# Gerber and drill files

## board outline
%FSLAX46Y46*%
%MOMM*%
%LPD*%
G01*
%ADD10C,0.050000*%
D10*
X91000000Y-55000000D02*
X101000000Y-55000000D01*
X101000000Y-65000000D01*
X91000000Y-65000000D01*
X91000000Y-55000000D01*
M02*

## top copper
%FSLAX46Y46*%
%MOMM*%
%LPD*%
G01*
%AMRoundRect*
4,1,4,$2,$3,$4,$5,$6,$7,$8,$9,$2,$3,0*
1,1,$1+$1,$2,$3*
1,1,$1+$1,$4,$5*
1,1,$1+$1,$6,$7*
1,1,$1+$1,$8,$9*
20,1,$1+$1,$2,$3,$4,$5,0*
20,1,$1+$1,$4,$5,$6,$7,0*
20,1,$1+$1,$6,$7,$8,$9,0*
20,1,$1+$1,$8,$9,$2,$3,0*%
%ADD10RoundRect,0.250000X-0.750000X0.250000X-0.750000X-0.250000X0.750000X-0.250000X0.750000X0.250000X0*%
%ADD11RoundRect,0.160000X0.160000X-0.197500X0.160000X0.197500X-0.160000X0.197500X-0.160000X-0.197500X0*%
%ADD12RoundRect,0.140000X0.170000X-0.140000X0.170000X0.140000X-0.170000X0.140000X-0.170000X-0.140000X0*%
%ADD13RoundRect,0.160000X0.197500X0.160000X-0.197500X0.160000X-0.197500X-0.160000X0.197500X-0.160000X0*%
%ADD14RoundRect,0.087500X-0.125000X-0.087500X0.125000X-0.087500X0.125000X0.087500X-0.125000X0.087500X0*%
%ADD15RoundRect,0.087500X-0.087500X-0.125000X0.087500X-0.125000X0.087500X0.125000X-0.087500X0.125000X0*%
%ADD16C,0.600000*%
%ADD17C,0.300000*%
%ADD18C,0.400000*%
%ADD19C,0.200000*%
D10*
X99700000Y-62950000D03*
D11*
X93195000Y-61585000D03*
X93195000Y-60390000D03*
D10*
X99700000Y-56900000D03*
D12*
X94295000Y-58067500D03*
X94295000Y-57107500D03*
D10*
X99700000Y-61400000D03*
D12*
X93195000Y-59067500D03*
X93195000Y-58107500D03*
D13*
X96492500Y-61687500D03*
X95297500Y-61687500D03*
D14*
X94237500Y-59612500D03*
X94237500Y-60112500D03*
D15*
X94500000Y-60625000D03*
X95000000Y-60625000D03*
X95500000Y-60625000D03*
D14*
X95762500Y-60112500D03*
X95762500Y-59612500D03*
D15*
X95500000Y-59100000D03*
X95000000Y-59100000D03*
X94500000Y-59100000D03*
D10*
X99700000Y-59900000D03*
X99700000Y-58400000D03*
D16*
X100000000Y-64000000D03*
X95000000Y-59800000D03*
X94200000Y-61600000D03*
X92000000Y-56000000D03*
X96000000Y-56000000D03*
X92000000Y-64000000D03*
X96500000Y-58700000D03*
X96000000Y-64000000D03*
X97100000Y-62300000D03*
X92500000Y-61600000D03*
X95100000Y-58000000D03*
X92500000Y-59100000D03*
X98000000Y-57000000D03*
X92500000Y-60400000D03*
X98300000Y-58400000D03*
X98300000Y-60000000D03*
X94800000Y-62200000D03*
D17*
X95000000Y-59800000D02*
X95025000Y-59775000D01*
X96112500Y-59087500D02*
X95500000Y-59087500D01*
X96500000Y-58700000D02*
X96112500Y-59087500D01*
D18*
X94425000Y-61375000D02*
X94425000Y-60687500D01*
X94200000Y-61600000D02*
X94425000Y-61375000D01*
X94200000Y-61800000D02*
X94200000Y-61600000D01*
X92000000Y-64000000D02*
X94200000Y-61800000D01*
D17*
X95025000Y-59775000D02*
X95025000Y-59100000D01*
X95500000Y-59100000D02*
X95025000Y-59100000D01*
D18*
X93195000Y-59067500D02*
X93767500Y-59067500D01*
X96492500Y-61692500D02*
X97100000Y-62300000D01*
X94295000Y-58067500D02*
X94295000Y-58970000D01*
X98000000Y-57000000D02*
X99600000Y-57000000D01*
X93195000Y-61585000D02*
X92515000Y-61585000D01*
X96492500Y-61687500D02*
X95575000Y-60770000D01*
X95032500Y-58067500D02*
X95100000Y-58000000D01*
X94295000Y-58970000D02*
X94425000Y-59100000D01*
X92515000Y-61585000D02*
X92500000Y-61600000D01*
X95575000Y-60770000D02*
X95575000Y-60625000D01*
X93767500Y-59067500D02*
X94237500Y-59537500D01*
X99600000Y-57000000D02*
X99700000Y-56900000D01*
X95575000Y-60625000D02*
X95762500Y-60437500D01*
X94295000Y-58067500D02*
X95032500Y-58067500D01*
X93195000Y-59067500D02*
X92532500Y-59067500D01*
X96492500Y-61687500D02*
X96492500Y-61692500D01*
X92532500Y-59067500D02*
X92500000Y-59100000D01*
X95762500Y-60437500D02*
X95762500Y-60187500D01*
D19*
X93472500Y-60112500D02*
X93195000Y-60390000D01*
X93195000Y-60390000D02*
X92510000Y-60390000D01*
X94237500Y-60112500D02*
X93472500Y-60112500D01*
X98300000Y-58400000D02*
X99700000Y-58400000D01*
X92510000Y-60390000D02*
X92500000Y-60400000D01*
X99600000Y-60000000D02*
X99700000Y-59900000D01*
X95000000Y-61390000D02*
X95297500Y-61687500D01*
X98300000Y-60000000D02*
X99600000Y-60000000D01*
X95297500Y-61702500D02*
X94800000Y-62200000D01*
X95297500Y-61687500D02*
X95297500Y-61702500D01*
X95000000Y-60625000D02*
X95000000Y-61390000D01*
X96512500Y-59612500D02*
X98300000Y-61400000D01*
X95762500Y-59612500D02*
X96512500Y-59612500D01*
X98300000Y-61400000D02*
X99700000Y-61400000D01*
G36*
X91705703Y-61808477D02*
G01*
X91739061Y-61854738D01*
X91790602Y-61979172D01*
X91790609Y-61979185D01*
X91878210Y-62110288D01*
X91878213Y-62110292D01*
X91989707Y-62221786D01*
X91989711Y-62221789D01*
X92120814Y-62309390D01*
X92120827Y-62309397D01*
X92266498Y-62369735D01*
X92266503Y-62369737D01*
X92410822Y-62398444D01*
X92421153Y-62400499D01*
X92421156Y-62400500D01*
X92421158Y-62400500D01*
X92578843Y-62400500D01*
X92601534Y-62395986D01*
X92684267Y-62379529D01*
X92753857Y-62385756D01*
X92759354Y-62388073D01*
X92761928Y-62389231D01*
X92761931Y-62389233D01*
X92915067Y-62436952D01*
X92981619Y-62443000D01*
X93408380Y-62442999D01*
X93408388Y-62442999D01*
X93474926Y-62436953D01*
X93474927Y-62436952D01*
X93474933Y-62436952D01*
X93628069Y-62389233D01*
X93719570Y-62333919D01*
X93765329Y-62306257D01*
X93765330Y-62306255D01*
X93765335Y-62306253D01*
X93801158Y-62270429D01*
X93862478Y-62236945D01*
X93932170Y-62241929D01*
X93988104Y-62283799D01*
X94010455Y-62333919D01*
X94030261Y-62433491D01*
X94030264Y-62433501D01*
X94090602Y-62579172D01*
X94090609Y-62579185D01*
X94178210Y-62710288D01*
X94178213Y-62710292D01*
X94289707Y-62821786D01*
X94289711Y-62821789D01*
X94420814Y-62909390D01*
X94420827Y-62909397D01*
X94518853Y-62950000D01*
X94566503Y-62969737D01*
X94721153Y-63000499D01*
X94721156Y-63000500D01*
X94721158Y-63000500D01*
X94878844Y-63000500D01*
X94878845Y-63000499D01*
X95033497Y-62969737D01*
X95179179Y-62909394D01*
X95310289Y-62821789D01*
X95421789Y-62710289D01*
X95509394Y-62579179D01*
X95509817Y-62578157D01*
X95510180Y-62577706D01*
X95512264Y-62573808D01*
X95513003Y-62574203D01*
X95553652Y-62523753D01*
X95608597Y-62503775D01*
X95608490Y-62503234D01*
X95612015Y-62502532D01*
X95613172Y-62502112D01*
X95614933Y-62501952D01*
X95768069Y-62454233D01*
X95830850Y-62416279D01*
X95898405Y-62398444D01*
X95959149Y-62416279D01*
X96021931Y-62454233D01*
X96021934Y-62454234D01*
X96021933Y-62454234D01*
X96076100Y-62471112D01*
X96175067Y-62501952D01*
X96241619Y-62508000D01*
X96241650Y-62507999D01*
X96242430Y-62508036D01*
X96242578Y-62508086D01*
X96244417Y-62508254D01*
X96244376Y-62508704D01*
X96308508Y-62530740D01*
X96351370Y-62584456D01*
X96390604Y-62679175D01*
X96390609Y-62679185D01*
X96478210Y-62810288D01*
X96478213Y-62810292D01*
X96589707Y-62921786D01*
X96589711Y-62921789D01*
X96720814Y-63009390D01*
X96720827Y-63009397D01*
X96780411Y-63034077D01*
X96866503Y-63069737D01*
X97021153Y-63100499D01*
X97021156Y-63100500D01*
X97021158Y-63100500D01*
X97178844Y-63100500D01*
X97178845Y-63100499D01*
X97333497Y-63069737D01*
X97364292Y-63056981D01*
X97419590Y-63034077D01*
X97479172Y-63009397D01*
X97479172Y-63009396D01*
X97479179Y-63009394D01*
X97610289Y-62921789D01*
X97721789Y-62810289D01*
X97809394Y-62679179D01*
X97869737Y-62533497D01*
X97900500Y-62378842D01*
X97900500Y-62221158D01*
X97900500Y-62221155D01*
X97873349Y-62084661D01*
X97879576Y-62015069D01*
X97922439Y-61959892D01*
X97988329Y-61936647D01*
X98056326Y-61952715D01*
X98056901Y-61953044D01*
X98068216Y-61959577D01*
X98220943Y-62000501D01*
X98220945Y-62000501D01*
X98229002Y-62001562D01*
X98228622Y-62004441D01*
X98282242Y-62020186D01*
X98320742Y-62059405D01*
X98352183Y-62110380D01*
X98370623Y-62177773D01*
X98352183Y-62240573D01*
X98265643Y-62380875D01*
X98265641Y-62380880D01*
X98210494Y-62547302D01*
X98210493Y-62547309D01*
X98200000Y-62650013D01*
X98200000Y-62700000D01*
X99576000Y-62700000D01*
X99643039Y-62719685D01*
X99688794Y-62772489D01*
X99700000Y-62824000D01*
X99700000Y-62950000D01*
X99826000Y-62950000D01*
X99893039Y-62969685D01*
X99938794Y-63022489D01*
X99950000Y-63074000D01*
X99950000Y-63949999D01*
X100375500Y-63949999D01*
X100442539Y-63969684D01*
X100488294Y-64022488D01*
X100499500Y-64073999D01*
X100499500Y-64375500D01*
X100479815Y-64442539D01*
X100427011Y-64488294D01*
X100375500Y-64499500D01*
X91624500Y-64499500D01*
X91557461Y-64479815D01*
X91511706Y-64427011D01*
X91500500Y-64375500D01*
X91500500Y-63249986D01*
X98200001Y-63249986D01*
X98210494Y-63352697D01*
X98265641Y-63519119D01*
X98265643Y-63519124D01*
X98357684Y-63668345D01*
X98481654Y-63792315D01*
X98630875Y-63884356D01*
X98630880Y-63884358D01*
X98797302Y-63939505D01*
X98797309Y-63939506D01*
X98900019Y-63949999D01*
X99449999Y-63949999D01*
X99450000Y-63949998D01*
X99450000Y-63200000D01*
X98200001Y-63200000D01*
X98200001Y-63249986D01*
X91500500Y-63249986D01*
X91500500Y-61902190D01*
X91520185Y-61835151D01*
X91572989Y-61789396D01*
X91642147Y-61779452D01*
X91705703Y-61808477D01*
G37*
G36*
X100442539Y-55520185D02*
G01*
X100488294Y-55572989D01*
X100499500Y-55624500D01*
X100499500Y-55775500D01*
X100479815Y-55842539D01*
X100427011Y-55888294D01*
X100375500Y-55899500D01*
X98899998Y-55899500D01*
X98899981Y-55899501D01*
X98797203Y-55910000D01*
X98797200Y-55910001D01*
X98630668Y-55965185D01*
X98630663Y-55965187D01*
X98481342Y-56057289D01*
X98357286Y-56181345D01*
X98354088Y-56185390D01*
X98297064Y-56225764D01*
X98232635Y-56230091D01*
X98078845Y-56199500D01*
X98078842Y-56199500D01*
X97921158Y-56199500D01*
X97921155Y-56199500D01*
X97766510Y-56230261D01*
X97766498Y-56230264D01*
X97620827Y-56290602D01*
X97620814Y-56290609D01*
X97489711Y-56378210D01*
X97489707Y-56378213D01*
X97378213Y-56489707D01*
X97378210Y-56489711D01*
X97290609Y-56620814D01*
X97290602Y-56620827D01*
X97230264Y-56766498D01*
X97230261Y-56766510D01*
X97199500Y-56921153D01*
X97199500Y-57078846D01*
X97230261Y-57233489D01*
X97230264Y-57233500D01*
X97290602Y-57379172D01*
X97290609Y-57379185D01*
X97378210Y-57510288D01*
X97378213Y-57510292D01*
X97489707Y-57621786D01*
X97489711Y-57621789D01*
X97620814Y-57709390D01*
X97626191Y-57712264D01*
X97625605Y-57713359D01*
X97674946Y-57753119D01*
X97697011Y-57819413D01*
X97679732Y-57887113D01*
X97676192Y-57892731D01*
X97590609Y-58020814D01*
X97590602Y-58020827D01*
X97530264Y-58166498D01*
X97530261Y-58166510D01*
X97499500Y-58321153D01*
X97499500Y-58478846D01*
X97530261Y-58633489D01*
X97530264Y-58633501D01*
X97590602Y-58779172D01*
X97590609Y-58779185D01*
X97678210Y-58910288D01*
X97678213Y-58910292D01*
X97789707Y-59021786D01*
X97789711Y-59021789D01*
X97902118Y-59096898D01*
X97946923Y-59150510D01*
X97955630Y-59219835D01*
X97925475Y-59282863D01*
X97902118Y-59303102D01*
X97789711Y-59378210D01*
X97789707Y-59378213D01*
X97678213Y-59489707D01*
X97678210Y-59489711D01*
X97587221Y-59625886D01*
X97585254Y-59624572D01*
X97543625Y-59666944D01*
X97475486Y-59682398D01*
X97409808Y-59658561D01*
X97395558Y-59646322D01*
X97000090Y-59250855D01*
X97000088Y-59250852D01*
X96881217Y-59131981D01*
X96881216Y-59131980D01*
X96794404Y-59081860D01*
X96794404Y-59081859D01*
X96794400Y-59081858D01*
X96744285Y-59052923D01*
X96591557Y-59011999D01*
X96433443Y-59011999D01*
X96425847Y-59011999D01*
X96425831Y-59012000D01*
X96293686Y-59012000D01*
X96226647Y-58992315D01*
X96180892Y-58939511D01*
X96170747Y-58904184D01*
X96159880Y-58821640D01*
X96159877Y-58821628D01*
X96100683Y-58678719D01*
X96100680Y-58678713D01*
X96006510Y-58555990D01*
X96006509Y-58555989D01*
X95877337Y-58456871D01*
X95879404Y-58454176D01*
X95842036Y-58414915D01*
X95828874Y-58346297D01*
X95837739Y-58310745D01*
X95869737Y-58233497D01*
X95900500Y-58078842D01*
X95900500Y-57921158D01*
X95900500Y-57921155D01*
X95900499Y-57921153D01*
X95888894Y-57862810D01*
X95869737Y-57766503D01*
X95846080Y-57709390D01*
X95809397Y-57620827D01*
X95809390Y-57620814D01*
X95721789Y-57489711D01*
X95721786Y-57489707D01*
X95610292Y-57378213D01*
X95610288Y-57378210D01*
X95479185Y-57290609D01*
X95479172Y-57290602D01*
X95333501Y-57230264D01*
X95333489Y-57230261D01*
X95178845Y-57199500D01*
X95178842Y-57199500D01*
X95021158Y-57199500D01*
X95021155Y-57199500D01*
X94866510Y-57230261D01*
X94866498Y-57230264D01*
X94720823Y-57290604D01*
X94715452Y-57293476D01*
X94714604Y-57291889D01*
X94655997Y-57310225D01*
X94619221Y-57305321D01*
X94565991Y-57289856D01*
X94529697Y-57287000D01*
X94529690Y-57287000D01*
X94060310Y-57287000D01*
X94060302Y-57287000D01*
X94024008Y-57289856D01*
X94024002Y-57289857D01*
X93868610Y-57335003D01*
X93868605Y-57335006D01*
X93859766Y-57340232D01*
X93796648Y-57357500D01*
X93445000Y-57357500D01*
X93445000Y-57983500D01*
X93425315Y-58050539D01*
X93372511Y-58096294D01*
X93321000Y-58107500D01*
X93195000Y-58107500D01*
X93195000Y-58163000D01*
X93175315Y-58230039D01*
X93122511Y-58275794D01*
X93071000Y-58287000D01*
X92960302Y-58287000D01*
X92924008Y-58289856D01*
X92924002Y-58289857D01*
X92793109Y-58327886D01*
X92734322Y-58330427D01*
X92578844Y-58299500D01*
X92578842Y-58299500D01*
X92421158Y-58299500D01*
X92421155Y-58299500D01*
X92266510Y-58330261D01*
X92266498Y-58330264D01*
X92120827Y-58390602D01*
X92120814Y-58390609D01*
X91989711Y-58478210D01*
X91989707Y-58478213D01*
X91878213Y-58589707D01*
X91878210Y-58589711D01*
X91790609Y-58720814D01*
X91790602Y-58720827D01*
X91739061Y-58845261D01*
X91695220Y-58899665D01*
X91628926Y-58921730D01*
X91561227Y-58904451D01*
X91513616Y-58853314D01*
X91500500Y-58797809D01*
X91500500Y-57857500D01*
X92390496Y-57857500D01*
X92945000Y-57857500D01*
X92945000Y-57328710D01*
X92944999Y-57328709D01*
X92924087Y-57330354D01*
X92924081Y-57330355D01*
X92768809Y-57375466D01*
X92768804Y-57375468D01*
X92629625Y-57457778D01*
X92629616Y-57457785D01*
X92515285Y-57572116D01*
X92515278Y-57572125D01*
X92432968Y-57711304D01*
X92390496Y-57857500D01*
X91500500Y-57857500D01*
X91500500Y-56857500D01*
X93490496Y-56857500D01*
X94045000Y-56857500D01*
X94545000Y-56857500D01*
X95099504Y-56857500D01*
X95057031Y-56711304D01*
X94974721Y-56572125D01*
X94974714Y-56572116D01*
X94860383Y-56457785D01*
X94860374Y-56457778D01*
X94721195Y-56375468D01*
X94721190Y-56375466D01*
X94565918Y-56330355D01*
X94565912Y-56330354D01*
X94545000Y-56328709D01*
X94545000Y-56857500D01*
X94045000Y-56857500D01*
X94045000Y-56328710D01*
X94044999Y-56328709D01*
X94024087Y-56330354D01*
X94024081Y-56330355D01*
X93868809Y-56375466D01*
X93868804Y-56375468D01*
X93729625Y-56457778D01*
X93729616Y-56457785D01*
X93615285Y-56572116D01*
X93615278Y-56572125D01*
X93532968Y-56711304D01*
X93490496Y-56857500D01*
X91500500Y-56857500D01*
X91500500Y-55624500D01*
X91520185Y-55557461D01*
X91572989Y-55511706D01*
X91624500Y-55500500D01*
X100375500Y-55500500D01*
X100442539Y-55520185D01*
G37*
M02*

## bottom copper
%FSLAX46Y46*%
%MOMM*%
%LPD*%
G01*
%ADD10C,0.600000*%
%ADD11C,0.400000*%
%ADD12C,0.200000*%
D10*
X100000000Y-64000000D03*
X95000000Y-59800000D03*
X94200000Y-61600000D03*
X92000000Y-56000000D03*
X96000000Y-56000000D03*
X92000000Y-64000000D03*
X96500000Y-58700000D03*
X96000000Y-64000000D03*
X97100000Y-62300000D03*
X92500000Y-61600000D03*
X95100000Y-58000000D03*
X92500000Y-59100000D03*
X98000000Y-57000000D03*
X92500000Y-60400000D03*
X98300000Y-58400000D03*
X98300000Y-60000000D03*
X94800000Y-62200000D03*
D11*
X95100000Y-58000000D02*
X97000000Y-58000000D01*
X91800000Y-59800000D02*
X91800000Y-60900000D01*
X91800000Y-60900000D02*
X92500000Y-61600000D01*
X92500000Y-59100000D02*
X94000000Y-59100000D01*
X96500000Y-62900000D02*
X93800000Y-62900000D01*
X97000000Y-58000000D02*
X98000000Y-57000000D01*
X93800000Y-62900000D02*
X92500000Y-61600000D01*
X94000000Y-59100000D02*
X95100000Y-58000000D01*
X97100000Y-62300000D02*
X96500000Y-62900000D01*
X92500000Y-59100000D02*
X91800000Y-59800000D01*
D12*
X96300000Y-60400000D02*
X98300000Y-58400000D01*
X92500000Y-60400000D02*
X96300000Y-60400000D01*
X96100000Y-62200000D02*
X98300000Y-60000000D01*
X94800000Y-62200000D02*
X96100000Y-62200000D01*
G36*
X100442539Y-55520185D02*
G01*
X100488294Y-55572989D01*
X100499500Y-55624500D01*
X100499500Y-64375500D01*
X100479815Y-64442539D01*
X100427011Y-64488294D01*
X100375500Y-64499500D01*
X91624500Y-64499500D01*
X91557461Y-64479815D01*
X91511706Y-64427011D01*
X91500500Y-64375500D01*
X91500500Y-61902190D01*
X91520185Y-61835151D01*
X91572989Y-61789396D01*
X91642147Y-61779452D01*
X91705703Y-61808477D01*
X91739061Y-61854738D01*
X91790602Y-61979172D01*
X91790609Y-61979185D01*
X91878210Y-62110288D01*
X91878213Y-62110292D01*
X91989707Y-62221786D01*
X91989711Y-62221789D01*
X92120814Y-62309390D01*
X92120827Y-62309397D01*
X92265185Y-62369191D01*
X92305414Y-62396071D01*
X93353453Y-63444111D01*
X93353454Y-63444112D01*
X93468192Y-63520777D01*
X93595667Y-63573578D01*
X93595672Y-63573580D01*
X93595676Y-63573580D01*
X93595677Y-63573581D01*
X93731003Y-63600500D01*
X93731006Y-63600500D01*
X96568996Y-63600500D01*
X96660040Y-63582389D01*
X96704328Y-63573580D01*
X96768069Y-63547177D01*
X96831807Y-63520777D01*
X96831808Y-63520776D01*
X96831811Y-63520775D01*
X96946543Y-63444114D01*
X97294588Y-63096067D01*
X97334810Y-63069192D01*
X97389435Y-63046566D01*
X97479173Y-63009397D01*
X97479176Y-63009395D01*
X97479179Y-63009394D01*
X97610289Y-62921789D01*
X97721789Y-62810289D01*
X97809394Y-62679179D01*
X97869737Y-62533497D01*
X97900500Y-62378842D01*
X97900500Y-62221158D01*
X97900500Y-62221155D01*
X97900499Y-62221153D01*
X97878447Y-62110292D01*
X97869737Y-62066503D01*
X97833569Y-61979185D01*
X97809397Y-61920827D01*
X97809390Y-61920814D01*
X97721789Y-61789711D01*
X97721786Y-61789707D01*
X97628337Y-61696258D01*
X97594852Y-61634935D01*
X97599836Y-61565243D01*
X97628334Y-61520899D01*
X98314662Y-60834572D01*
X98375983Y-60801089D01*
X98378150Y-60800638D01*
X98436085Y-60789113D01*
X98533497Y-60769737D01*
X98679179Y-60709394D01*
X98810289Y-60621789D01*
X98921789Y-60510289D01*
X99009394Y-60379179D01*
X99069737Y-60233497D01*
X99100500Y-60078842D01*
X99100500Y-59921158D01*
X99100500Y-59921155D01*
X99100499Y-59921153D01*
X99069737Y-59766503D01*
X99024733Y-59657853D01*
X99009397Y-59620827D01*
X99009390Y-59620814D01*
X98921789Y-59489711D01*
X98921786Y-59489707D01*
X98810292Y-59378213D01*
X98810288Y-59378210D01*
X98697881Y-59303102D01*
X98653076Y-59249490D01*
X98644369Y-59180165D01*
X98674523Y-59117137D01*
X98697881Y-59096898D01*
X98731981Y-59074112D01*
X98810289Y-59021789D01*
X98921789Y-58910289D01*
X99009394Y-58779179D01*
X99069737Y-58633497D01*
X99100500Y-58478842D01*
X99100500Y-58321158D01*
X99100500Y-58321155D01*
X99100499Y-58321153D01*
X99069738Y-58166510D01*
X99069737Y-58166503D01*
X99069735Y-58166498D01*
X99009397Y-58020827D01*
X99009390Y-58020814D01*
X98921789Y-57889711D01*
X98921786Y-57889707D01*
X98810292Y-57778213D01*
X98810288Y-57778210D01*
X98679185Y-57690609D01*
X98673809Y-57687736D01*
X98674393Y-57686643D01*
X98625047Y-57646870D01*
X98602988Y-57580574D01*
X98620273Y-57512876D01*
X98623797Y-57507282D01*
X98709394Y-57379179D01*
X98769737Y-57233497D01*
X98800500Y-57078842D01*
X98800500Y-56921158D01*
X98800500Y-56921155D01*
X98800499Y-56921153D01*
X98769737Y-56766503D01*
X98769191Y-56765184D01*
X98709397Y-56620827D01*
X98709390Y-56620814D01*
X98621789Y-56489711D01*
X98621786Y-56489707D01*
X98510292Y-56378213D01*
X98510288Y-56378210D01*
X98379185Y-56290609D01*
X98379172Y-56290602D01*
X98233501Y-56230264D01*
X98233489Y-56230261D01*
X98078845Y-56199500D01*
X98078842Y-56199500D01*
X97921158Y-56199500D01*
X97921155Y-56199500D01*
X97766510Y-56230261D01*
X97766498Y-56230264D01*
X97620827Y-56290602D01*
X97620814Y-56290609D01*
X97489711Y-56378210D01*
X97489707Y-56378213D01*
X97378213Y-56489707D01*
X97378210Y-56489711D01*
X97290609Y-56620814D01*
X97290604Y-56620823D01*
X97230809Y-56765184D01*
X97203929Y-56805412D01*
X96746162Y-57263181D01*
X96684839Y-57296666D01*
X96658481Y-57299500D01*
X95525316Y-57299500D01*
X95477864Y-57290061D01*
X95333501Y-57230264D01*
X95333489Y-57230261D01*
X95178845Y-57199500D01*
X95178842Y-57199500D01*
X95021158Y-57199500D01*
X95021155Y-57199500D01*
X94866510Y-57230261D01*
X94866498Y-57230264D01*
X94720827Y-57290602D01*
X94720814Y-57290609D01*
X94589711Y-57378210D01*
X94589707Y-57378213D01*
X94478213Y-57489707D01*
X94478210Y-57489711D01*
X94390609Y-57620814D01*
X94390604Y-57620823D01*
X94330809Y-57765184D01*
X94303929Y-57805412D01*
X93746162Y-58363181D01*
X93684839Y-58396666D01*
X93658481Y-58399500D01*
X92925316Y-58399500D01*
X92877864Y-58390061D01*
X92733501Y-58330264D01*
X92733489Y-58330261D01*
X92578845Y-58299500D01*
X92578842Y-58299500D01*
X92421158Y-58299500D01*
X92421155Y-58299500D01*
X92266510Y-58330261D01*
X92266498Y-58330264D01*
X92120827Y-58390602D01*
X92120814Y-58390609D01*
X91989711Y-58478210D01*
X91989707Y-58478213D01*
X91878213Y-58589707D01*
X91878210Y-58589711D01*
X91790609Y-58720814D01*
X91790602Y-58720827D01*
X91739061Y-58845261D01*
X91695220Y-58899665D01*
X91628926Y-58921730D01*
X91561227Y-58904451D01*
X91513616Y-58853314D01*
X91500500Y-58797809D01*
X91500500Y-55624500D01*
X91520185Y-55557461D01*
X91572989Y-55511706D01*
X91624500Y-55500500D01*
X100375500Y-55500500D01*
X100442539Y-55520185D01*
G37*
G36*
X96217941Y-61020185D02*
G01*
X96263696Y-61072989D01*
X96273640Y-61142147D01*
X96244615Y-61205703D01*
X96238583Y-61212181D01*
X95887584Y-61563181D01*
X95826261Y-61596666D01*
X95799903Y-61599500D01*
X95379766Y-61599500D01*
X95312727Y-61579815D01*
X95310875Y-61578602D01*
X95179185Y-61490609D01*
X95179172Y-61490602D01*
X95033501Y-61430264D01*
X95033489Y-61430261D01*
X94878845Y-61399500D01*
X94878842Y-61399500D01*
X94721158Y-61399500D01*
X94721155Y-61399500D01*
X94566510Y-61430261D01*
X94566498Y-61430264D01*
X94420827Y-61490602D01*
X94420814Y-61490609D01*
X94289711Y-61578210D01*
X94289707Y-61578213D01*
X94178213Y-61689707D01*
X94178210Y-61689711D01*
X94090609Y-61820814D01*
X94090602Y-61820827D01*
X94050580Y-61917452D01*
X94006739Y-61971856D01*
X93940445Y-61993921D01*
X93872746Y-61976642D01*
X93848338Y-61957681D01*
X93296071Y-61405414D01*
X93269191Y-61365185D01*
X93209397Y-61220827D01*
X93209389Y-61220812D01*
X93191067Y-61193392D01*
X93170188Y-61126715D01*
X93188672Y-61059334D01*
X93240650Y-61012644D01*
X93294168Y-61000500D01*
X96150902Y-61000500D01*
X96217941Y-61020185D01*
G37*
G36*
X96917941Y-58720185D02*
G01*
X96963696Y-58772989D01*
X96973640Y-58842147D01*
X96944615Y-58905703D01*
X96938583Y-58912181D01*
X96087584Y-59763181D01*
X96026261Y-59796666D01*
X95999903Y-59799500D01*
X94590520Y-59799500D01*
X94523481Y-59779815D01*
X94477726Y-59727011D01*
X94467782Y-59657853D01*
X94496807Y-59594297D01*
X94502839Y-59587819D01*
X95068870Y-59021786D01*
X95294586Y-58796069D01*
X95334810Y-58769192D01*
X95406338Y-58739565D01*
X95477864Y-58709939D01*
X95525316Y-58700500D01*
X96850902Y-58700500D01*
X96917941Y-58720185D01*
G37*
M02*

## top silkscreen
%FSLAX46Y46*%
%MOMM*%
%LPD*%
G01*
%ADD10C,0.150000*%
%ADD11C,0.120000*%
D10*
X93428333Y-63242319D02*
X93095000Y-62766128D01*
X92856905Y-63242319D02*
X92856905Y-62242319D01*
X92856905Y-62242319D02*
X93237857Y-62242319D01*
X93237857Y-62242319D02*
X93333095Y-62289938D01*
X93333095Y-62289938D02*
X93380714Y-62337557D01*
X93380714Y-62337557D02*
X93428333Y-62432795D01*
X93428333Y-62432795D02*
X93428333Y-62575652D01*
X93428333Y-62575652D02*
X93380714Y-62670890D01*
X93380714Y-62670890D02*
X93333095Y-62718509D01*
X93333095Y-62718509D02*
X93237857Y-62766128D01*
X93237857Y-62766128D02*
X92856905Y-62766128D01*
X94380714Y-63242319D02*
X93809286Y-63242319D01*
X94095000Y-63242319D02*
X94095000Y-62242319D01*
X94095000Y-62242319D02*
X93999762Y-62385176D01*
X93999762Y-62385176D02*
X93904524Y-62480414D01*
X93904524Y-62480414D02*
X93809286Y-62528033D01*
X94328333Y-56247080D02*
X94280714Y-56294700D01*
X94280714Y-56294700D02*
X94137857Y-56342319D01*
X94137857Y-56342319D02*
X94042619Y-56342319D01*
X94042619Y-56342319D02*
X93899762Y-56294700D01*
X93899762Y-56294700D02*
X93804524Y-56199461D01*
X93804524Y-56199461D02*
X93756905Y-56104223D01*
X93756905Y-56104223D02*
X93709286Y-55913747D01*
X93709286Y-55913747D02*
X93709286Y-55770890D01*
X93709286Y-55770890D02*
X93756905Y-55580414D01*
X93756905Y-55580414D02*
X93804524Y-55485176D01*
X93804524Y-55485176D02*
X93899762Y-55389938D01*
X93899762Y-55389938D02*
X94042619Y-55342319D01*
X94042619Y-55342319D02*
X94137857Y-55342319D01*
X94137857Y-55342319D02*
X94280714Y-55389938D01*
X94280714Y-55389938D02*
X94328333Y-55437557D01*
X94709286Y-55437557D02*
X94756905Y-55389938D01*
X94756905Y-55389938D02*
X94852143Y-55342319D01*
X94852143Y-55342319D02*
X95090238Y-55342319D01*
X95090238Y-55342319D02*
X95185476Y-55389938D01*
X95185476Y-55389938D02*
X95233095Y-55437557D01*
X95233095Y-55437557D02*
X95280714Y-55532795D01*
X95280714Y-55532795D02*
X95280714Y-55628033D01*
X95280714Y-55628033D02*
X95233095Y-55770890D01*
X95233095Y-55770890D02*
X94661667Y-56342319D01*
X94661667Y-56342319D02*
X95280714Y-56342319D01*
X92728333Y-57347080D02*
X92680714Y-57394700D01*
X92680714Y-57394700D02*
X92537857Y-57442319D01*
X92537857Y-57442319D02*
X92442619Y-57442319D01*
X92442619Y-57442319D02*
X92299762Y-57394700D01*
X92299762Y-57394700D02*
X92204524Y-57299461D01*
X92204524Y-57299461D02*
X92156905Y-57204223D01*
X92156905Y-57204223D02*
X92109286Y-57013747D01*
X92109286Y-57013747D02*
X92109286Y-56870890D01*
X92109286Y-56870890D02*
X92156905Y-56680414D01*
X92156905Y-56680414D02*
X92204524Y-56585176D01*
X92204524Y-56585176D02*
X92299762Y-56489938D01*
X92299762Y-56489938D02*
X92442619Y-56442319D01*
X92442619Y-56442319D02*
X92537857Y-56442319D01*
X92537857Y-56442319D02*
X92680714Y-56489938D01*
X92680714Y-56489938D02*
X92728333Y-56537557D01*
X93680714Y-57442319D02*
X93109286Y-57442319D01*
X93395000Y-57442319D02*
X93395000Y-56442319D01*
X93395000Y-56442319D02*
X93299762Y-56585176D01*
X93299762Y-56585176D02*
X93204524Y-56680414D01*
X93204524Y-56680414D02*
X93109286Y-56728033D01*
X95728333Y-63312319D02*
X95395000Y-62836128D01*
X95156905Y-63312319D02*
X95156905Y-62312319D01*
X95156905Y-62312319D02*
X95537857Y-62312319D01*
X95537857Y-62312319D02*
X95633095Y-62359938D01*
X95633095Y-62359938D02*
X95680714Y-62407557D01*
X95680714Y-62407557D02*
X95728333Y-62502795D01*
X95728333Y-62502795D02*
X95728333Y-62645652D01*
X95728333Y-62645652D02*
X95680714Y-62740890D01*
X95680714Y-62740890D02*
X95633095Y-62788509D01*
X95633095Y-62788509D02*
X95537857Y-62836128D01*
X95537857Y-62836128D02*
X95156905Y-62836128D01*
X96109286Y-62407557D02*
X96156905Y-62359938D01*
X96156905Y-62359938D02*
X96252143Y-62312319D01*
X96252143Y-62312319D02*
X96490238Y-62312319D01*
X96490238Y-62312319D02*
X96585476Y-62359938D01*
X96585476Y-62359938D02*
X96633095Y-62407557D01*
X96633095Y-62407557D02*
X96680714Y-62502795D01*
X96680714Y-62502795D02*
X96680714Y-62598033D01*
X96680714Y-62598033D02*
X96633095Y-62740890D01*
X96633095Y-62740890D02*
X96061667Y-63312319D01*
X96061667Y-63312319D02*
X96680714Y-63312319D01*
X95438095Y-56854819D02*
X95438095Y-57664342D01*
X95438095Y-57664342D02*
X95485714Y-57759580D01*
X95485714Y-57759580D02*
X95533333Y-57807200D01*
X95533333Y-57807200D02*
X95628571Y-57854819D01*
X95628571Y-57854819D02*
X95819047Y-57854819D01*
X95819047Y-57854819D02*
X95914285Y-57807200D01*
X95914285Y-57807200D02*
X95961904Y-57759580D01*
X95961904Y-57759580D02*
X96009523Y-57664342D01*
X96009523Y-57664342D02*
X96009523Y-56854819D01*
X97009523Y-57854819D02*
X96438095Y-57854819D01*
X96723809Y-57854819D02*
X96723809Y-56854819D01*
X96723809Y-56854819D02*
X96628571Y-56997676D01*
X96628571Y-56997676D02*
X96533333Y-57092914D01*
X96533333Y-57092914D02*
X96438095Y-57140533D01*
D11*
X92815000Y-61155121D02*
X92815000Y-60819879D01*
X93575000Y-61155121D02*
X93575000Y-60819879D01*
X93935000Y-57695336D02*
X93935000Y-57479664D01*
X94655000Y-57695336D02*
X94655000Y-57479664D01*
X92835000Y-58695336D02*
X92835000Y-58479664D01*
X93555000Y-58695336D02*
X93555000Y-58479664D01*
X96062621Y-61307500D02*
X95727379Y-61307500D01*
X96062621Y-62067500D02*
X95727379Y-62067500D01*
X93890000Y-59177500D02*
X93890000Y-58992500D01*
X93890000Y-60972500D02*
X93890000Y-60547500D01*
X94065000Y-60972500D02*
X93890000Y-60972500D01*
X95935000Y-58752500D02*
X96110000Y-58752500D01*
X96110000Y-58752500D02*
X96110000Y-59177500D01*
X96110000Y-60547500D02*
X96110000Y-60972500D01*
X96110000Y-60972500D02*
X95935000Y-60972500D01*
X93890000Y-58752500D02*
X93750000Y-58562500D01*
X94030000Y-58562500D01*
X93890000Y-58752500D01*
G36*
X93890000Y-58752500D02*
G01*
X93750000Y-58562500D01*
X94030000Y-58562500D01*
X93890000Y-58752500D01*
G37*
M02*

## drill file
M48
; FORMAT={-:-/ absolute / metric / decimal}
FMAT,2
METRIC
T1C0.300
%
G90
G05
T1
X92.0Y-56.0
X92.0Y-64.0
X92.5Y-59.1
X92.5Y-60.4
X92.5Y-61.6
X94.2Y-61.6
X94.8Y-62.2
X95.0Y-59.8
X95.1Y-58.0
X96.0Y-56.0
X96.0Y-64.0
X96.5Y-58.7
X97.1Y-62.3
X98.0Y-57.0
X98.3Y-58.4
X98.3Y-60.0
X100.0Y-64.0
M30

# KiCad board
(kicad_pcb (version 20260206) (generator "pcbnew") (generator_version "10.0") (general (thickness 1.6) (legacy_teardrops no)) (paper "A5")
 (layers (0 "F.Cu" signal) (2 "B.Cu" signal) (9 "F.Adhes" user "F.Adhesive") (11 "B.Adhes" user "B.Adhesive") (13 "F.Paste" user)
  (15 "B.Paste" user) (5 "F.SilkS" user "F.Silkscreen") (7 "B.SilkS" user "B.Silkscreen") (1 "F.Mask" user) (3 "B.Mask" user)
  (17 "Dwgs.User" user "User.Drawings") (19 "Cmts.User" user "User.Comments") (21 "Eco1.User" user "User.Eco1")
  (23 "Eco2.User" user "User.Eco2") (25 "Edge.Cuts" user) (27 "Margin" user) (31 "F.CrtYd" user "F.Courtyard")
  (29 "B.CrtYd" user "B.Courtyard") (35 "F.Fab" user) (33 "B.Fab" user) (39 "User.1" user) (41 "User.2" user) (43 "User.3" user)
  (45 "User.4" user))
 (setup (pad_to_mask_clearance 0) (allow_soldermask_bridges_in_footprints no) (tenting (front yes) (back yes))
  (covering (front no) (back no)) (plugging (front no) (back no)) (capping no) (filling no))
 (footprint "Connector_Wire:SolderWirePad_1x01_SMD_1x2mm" (layer "F.Cu") (at 99.7 62.95 -90)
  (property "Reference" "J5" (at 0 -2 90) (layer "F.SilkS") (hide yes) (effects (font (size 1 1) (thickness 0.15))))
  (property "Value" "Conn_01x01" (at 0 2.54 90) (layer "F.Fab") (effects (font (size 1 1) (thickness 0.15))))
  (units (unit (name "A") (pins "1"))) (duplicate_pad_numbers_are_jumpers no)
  (pad "1" smd roundrect (at 0 0 270) (size 1 2) (layers "F.Cu" "F.Mask") (roundrect_rratio 0.25) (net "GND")))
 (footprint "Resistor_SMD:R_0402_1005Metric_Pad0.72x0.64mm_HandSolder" (layer "F.Cu") (at 93.195 60.9875 90)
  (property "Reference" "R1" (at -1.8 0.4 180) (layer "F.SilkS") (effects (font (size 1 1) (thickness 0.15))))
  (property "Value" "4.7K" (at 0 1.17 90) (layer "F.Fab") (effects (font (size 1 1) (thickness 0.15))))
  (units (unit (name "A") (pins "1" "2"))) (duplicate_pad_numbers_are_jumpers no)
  (fp_line (start -0.167621 -0.38) (end 0.167621 -0.38) (stroke (width 0.12) (type solid)) (layer "F.SilkS"))
  (fp_line (start -0.167621 0.38) (end 0.167621 0.38) (stroke (width 0.12) (type solid)) (layer "F.SilkS"))
  (pad "1" smd roundrect (at -0.5975 0 90) (size 0.715 0.64) (layers "F.Cu" "F.Mask" "F.Paste") (roundrect_rratio 0.25) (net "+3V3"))
  (pad "2" smd roundrect (at 0.5975 0 90) (size 0.715 0.64) (layers "F.Cu" "F.Mask" "F.Paste") (roundrect_rratio 0.25) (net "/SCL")))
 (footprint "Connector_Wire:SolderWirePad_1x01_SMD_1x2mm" (layer "F.Cu") (at 99.7 56.9 -90)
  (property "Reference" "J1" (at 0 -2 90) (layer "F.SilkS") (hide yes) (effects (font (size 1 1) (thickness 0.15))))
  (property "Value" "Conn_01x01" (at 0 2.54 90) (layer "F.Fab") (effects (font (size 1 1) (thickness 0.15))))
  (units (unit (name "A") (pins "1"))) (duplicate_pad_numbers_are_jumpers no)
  (pad "1" smd roundrect (at 0 0 270) (size 1 2) (layers "F.Cu" "F.Mask") (roundrect_rratio 0.25) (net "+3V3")))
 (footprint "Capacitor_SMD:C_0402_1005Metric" (layer "F.Cu") (at 94.295 57.5875 90)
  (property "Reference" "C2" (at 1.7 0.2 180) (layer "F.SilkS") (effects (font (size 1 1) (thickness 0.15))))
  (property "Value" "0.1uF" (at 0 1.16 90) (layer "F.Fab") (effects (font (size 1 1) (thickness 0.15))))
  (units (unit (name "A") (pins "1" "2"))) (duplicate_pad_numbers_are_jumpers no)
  (fp_line (start -0.107836 -0.36) (end 0.107836 -0.36) (stroke (width 0.12) (type solid)) (layer "F.SilkS"))
  (fp_line (start -0.107836 0.36) (end 0.107836 0.36) (stroke (width 0.12) (type solid)) (layer "F.SilkS"))
  (pad "1" smd roundrect (at -0.48 0 90) (size 0.56 0.62) (layers "F.Cu" "F.Mask" "F.Paste") (roundrect_rratio 0.25) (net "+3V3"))
  (pad "2" smd roundrect (at 0.48 0 90) (size 0.56 0.62) (layers "F.Cu" "F.Mask" "F.Paste") (roundrect_rratio 0.25) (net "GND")))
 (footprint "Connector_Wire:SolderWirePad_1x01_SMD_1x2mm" (layer "F.Cu") (at 99.7 61.4 -90)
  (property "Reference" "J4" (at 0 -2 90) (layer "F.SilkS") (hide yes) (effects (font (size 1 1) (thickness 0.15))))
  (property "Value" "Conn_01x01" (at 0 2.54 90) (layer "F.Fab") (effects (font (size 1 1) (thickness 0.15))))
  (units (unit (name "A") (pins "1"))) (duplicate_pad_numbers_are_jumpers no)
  (pad "1" smd roundrect (at 0 0 270) (size 1 2) (layers "F.Cu" "F.Mask") (roundrect_rratio 0.25) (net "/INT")))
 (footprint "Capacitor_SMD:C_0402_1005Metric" (layer "F.Cu") (at 93.195 58.5875 90)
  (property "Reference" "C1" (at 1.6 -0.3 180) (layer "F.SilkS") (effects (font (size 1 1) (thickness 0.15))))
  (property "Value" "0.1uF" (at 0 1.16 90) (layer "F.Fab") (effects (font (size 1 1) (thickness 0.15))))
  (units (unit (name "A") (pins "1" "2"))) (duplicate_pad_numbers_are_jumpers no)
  (fp_line (start -0.107836 -0.36) (end 0.107836 -0.36) (stroke (width 0.12) (type solid)) (layer "F.SilkS"))
  (fp_line (start -0.107836 0.36) (end 0.107836 0.36) (stroke (width 0.12) (type solid)) (layer "F.SilkS"))
  (pad "1" smd roundrect (at -0.48 0 90) (size 0.56 0.62) (layers "F.Cu" "F.Mask" "F.Paste") (roundrect_rratio 0.25) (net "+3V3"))
  (pad "2" smd roundrect (at 0.48 0 90) (size 0.56 0.62) (layers "F.Cu" "F.Mask" "F.Paste") (roundrect_rratio 0.25) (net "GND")))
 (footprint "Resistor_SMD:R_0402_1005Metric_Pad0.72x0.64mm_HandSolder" (layer "F.Cu") (at 95.895 61.6875 180)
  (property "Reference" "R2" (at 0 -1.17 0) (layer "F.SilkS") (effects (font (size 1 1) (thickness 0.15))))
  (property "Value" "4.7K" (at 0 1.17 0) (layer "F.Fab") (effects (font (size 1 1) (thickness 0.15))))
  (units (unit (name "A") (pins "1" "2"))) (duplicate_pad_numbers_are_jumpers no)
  (fp_line (start -0.167621 0.38) (end 0.167621 0.38) (stroke (width 0.12) (type solid)) (layer "F.SilkS"))
  (fp_line (start -0.167621 -0.38) (end 0.167621 -0.38) (stroke (width 0.12) (type solid)) (layer "F.SilkS"))
  (pad "1" smd roundrect (at -0.5975 0 180) (size 0.715 0.64) (layers "F.Cu" "F.Mask" "F.Paste") (roundrect_rratio 0.25) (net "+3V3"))
  (pad "2" smd roundrect (at 0.5975 0 180) (size 0.715 0.64) (layers "F.Cu" "F.Mask" "F.Paste") (roundrect_rratio 0.25) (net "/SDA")))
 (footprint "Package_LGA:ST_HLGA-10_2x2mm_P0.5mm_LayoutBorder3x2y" (layer "F.Cu") (at 95 59.8625)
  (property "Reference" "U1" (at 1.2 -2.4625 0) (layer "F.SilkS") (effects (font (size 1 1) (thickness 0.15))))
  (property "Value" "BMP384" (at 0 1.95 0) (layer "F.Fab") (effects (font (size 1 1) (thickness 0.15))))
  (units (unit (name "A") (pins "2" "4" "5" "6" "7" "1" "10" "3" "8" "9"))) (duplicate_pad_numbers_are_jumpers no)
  (fp_line (start -1.11 -0.685) (end -1.11 -0.87) (stroke (width 0.12) (type solid)) (layer "F.SilkS"))
  (fp_line (start -1.11 1.11) (end -1.11 0.685) (stroke (width 0.12) (type solid)) (layer "F.SilkS"))
  (fp_line (start -0.935 1.11) (end -1.11 1.11) (stroke (width 0.12) (type solid)) (layer "F.SilkS"))
  (fp_line (start 0.935 -1.11) (end 1.11 -1.11) (stroke (width 0.12) (type solid)) (layer "F.SilkS"))
  (fp_line (start 1.11 -1.11) (end 1.11 -0.685) (stroke (width 0.12) (type solid)) (layer "F.SilkS"))
  (fp_line (start 1.11 0.685) (end 1.11 1.11) (stroke (width 0.12) (type solid)) (layer "F.SilkS"))
  (fp_line (start 1.11 1.11) (end 0.935 1.11) (stroke (width 0.12) (type solid)) (layer "F.SilkS"))
  (fp_poly (pts (xy -1.11 -1.11) (xy -1.25 -1.3) (xy -0.97 -1.3)) (stroke (width 0.12) (type solid)) (fill yes) (layer "F.SilkS"))
  (pad "1" smd roundrect (at -0.7625 -0.25) (size 0.425 0.35) (layers "F.Cu" "F.Mask" "F.Paste") (roundrect_rratio 0.25) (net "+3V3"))
  (pad "2" smd roundrect (at -0.7625 0.25) (size 0.425 0.35) (layers "F.Cu" "F.Mask" "F.Paste") (roundrect_rratio 0.25) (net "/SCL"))
  (pad "3" smd roundrect (at -0.5 0.7625) (size 0.35 0.425) (layers "F.Cu" "F.Mask" "F.Paste") (roundrect_rratio 0.25) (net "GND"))
  (pad "4" smd roundrect (at 0 0.7625) (size 0.35 0.425) (layers "F.Cu" "F.Mask" "F.Paste") (roundrect_rratio 0.25) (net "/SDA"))
  (pad "5" smd roundrect (at 0.5 0.7625) (size 0.35 0.425) (layers "F.Cu" "F.Mask" "F.Paste") (roundrect_rratio 0.25) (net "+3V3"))
  (pad "6" smd roundrect (at 0.7625 0.25) (size 0.425 0.35) (layers "F.Cu" "F.Mask" "F.Paste") (roundrect_rratio 0.25) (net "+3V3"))
  (pad "7" smd roundrect (at 0.7625 -0.25) (size 0.425 0.35) (layers "F.Cu" "F.Mask" "F.Paste") (roundrect_rratio 0.25) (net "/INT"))
  (pad "8" smd roundrect (at 0.5 -0.7625) (size 0.35 0.425) (layers "F.Cu" "F.Mask" "F.Paste") (roundrect_rratio 0.25) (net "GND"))
  (pad "9" smd roundrect (at 0 -0.7625) (size 0.35 0.425) (layers "F.Cu" "F.Mask" "F.Paste") (roundrect_rratio 0.25) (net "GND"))
  (pad "10" smd roundrect (at -0.5 -0.7625) (size 0.35 0.425) (layers "F.Cu" "F.Mask" "F.Paste") (roundrect_rratio 0.25) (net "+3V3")))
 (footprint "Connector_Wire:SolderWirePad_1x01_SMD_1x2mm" (layer "F.Cu") (at 99.7 59.9 -90)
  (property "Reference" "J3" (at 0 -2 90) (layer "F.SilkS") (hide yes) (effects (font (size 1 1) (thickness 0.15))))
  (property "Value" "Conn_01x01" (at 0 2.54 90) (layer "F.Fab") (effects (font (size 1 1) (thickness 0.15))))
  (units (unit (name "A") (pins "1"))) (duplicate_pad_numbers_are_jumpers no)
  (pad "1" smd roundrect (at 0 0 270) (size 1 2) (layers "F.Cu" "F.Mask") (roundrect_rratio 0.25) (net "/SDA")))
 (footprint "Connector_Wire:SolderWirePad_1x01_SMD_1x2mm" (layer "F.Cu") (at 99.7 58.4 -90)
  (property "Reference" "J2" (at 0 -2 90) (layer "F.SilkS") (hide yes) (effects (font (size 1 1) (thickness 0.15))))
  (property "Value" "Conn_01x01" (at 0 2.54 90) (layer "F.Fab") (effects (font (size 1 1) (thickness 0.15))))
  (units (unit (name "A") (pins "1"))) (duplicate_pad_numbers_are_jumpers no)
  (pad "1" smd roundrect (at 0 0 270) (size 1 2) (layers "F.Cu" "F.Mask") (roundrect_rratio 0.25) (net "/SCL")))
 (gr_rect (start 91 55) (end 101 65) (stroke (width 0.05) (type default)) (fill no) (layer "Edge.Cuts"))
 (segment (start 95 59.8) (end 95.025 59.775) (width 0.3) (layer "F.Cu") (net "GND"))
 (segment (start 96.1125 59.0875) (end 95.5 59.0875) (width 0.3) (layer "F.Cu") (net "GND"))
 (segment (start 96.5 58.7) (end 96.1125 59.0875) (width 0.3) (layer "F.Cu") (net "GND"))
 (segment (start 94.425 61.375) (end 94.425 60.6875) (width 0.4) (layer "F.Cu") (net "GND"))
 (segment (start 94.2 61.6) (end 94.425 61.375) (width 0.4) (layer "F.Cu") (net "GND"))
 (segment (start 94.2 61.8) (end 94.2 61.6) (width 0.4) (layer "F.Cu") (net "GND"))
 (segment (start 92 64) (end 94.2 61.8) (width 0.4) (layer "F.Cu") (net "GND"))
 (segment (start 95.025 59.775) (end 95.025 59.1) (width 0.3) (layer "F.Cu") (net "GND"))
 (segment (start 95.5 59.1) (end 95.025 59.1) (width 0.3) (layer "F.Cu") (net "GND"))
 (via (at 100 64) (size 0.6) (drill 0.3) (layers "F.Cu" "B.Cu") (free yes) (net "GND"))
 (via (at 95 59.8) (size 0.6) (drill 0.3) (layers "F.Cu" "B.Cu") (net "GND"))
 (via (at 94.2 61.6) (size 0.6) (drill 0.3) (layers "F.Cu" "B.Cu") (free yes) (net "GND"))
 (via (at 92 56) (size 0.6) (drill 0.3) (layers "F.Cu" "B.Cu") (free yes) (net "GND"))
 (via (at 96 56) (size 0.6) (drill 0.3) (layers "F.Cu" "B.Cu") (free yes) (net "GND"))
 (via (at 92 64) (size 0.6) (drill 0.3) (layers "F.Cu" "B.Cu") (free yes) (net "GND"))
 (via (at 96.5 58.7) (size 0.6) (drill 0.3) (layers "F.Cu" "B.Cu") (free yes) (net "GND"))
 (via (at 96 64) (size 0.6) (drill 0.3) (layers "F.Cu" "B.Cu") (free yes) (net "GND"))
 (segment (start 93.195 59.0675) (end 93.7675 59.0675) (width 0.4) (layer "F.Cu") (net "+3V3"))
 (segment (start 96.4925 61.6925) (end 97.1 62.3) (width 0.4) (layer "F.Cu") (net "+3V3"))
 (segment (start 94.295 58.0675) (end 94.295 58.97) (width 0.4) (layer "F.Cu") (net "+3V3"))
 (segment (start 98 57) (end 99.6 57) (width 0.4) (layer "F.Cu") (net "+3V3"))
 (segment (start 93.195 61.585) (end 92.515 61.585) (width 0.4) (layer "F.Cu") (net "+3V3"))
 (segment (start 96.4925 61.6875) (end 95.575 60.77) (width 0.4) (layer "F.Cu") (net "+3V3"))
 (segment (start 95.0325 58.0675) (end 95.1 58) (width 0.4) (layer "F.Cu") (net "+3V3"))
 (segment (start 94.295 58.97) (end 94.425 59.1) (width 0.4) (layer "F.Cu") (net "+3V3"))
 (segment (start 92.515 61.585) (end 92.5 61.6) (width 0.4) (layer "F.Cu") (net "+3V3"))
 (segment (start 95.575 60.77) (end 95.575 60.625) (width 0.4) (layer "F.Cu") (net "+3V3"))
 (segment (start 93.7675 59.0675) (end 94.2375 59.5375) (width 0.4) (layer "F.Cu") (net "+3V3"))
 (segment (start 99.6 57) (end 99.7 56.9) (width 0.4) (layer "F.Cu") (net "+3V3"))
 (segment (start 95.575 60.625) (end 95.7625 60.4375) (width 0.4) (layer "F.Cu") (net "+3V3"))
 (segment (start 94.295 58.0675) (end 95.0325 58.0675) (width 0.4) (layer "F.Cu") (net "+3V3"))
 (segment (start 93.195 59.0675) (end 92.5325 59.0675) (width 0.4) (layer "F.Cu") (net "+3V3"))
 (segment (start 96.4925 61.6875) (end 96.4925 61.6925) (width 0.4) (layer "F.Cu") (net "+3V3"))
 (segment (start 92.5325 59.0675) (end 92.5 59.1) (width 0.4) (layer "F.Cu") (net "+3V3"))
 (segment (start 95.7625 60.4375) (end 95.7625 60.1875) (width 0.4) (layer "F.Cu") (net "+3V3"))
 (via (at 97.1 62.3) (size 0.6) (drill 0.3) (layers "F.Cu" "B.Cu") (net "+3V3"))
 (via (at 92.5 61.6) (size 0.6) (drill 0.3) (layers "F.Cu" "B.Cu") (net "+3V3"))
 (via (at 95.1 58) (size 0.6) (drill 0.3) (layers "F.Cu" "B.Cu") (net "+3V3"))
 (via (at 92.5 59.1) (size 0.6) (drill 0.3) (layers "F.Cu" "B.Cu") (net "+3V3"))
 (via (at 98 57) (size 0.6) (drill 0.3) (layers "F.Cu" "B.Cu") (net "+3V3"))
 (segment (start 95.1 58) (end 97 58) (width 0.4) (layer "B.Cu") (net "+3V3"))
 (segment (start 91.8 59.8) (end 91.8 60.9) (width 0.4) (layer "B.Cu") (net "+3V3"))
 (segment (start 91.8 60.9) (end 92.5 61.6) (width 0.4) (layer "B.Cu") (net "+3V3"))
 (segment (start 92.5 59.1) (end 94 59.1) (width 0.4) (layer "B.Cu") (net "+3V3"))
 (segment (start 96.5 62.9) (end 93.8 62.9) (width 0.4) (layer "B.Cu") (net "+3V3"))
 (segment (start 97 58) (end 98 57) (width 0.4) (layer "B.Cu") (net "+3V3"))
 (segment (start 93.8 62.9) (end 92.5 61.6) (width 0.4) (layer "B.Cu") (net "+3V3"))
 (segment (start 94 59.1) (end 95.1 58) (width 0.4) (layer "B.Cu") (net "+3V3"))
 (segment (start 97.1 62.3) (end 96.5 62.9) (width 0.4) (layer "B.Cu") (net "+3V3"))
 (segment (start 92.5 59.1) (end 91.8 59.8) (width 0.4) (layer "B.Cu") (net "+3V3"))
 (segment (start 93.4725 60.1125) (end 93.195 60.39) (width 0.2) (layer "F.Cu") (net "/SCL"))
 (segment (start 93.195 60.39) (end 92.51 60.39) (width 0.2) (layer "F.Cu") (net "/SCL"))
 (segment (start 94.2375 60.1125) (end 93.4725 60.1125) (width 0.2) (layer "F.Cu") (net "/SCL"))
 (segment (start 98.3 58.4) (end 99.7 58.4) (width 0.2) (layer "F.Cu") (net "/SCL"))
 (segment (start 92.51 60.39) (end 92.5 60.4) (width 0.2) (layer "F.Cu") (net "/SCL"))
 (via (at 92.5 60.4) (size 0.6) (drill 0.3) (layers "F.Cu" "B.Cu") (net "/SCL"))
 (via (at 98.3 58.4) (size 0.6) (drill 0.3) (layers "F.Cu" "B.Cu") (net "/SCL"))
 (segment (start 96.3 60.4) (end 98.3 58.4) (width 0.2) (layer "B.Cu") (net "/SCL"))
 (segment (start 92.5 60.4) (end 96.3 60.4) (width 0.2) (layer "B.Cu") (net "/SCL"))
 (segment (start 99.6 60) (end 99.7 59.9) (width 0.2) (layer "F.Cu") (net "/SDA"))
 (segment (start 95 61.39) (end 95.2975 61.6875) (width 0.2) (layer "F.Cu") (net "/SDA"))
 (segment (start 98.3 60) (end 99.6 60) (width 0.2) (layer "F.Cu") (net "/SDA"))
 (segment (start 95.2975 61.7025) (end 94.8 62.2) (width 0.2) (layer "F.Cu") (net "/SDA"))
 (segment (start 95.2975 61.6875) (end 95.2975 61.7025) (width 0.2) (layer "F.Cu") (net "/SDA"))
 (segment (start 95 60.625) (end 95 61.39) (width 0.2) (layer "F.Cu") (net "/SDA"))
 (via (at 98.3 60) (size 0.6) (drill 0.3) (layers "F.Cu" "B.Cu") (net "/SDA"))
 (via (at 94.8 62.2) (size 0.6) (drill 0.3) (layers "F.Cu" "B.Cu") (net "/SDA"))
 (segment (start 96.1 62.2) (end 98.3 60) (width 0.2) (layer "B.Cu") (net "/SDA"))
 (segment (start 94.8 62.2) (end 96.1 62.2) (width 0.2) (layer "B.Cu") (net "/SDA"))
 (segment (start 96.5125 59.6125) (end 98.3 61.4) (width 0.2) (layer "F.Cu") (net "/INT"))
 (segment (start 95.7625 59.6125) (end 96.5125 59.6125) (width 0.2) (layer "F.Cu") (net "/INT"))
 (segment (start 98.3 61.4) (end 99.7 61.4) (width 0.2) (layer "F.Cu") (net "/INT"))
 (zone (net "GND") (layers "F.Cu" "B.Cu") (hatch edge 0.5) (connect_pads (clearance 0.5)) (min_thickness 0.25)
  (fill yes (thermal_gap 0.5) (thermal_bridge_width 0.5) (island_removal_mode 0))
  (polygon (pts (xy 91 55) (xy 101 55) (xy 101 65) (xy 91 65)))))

